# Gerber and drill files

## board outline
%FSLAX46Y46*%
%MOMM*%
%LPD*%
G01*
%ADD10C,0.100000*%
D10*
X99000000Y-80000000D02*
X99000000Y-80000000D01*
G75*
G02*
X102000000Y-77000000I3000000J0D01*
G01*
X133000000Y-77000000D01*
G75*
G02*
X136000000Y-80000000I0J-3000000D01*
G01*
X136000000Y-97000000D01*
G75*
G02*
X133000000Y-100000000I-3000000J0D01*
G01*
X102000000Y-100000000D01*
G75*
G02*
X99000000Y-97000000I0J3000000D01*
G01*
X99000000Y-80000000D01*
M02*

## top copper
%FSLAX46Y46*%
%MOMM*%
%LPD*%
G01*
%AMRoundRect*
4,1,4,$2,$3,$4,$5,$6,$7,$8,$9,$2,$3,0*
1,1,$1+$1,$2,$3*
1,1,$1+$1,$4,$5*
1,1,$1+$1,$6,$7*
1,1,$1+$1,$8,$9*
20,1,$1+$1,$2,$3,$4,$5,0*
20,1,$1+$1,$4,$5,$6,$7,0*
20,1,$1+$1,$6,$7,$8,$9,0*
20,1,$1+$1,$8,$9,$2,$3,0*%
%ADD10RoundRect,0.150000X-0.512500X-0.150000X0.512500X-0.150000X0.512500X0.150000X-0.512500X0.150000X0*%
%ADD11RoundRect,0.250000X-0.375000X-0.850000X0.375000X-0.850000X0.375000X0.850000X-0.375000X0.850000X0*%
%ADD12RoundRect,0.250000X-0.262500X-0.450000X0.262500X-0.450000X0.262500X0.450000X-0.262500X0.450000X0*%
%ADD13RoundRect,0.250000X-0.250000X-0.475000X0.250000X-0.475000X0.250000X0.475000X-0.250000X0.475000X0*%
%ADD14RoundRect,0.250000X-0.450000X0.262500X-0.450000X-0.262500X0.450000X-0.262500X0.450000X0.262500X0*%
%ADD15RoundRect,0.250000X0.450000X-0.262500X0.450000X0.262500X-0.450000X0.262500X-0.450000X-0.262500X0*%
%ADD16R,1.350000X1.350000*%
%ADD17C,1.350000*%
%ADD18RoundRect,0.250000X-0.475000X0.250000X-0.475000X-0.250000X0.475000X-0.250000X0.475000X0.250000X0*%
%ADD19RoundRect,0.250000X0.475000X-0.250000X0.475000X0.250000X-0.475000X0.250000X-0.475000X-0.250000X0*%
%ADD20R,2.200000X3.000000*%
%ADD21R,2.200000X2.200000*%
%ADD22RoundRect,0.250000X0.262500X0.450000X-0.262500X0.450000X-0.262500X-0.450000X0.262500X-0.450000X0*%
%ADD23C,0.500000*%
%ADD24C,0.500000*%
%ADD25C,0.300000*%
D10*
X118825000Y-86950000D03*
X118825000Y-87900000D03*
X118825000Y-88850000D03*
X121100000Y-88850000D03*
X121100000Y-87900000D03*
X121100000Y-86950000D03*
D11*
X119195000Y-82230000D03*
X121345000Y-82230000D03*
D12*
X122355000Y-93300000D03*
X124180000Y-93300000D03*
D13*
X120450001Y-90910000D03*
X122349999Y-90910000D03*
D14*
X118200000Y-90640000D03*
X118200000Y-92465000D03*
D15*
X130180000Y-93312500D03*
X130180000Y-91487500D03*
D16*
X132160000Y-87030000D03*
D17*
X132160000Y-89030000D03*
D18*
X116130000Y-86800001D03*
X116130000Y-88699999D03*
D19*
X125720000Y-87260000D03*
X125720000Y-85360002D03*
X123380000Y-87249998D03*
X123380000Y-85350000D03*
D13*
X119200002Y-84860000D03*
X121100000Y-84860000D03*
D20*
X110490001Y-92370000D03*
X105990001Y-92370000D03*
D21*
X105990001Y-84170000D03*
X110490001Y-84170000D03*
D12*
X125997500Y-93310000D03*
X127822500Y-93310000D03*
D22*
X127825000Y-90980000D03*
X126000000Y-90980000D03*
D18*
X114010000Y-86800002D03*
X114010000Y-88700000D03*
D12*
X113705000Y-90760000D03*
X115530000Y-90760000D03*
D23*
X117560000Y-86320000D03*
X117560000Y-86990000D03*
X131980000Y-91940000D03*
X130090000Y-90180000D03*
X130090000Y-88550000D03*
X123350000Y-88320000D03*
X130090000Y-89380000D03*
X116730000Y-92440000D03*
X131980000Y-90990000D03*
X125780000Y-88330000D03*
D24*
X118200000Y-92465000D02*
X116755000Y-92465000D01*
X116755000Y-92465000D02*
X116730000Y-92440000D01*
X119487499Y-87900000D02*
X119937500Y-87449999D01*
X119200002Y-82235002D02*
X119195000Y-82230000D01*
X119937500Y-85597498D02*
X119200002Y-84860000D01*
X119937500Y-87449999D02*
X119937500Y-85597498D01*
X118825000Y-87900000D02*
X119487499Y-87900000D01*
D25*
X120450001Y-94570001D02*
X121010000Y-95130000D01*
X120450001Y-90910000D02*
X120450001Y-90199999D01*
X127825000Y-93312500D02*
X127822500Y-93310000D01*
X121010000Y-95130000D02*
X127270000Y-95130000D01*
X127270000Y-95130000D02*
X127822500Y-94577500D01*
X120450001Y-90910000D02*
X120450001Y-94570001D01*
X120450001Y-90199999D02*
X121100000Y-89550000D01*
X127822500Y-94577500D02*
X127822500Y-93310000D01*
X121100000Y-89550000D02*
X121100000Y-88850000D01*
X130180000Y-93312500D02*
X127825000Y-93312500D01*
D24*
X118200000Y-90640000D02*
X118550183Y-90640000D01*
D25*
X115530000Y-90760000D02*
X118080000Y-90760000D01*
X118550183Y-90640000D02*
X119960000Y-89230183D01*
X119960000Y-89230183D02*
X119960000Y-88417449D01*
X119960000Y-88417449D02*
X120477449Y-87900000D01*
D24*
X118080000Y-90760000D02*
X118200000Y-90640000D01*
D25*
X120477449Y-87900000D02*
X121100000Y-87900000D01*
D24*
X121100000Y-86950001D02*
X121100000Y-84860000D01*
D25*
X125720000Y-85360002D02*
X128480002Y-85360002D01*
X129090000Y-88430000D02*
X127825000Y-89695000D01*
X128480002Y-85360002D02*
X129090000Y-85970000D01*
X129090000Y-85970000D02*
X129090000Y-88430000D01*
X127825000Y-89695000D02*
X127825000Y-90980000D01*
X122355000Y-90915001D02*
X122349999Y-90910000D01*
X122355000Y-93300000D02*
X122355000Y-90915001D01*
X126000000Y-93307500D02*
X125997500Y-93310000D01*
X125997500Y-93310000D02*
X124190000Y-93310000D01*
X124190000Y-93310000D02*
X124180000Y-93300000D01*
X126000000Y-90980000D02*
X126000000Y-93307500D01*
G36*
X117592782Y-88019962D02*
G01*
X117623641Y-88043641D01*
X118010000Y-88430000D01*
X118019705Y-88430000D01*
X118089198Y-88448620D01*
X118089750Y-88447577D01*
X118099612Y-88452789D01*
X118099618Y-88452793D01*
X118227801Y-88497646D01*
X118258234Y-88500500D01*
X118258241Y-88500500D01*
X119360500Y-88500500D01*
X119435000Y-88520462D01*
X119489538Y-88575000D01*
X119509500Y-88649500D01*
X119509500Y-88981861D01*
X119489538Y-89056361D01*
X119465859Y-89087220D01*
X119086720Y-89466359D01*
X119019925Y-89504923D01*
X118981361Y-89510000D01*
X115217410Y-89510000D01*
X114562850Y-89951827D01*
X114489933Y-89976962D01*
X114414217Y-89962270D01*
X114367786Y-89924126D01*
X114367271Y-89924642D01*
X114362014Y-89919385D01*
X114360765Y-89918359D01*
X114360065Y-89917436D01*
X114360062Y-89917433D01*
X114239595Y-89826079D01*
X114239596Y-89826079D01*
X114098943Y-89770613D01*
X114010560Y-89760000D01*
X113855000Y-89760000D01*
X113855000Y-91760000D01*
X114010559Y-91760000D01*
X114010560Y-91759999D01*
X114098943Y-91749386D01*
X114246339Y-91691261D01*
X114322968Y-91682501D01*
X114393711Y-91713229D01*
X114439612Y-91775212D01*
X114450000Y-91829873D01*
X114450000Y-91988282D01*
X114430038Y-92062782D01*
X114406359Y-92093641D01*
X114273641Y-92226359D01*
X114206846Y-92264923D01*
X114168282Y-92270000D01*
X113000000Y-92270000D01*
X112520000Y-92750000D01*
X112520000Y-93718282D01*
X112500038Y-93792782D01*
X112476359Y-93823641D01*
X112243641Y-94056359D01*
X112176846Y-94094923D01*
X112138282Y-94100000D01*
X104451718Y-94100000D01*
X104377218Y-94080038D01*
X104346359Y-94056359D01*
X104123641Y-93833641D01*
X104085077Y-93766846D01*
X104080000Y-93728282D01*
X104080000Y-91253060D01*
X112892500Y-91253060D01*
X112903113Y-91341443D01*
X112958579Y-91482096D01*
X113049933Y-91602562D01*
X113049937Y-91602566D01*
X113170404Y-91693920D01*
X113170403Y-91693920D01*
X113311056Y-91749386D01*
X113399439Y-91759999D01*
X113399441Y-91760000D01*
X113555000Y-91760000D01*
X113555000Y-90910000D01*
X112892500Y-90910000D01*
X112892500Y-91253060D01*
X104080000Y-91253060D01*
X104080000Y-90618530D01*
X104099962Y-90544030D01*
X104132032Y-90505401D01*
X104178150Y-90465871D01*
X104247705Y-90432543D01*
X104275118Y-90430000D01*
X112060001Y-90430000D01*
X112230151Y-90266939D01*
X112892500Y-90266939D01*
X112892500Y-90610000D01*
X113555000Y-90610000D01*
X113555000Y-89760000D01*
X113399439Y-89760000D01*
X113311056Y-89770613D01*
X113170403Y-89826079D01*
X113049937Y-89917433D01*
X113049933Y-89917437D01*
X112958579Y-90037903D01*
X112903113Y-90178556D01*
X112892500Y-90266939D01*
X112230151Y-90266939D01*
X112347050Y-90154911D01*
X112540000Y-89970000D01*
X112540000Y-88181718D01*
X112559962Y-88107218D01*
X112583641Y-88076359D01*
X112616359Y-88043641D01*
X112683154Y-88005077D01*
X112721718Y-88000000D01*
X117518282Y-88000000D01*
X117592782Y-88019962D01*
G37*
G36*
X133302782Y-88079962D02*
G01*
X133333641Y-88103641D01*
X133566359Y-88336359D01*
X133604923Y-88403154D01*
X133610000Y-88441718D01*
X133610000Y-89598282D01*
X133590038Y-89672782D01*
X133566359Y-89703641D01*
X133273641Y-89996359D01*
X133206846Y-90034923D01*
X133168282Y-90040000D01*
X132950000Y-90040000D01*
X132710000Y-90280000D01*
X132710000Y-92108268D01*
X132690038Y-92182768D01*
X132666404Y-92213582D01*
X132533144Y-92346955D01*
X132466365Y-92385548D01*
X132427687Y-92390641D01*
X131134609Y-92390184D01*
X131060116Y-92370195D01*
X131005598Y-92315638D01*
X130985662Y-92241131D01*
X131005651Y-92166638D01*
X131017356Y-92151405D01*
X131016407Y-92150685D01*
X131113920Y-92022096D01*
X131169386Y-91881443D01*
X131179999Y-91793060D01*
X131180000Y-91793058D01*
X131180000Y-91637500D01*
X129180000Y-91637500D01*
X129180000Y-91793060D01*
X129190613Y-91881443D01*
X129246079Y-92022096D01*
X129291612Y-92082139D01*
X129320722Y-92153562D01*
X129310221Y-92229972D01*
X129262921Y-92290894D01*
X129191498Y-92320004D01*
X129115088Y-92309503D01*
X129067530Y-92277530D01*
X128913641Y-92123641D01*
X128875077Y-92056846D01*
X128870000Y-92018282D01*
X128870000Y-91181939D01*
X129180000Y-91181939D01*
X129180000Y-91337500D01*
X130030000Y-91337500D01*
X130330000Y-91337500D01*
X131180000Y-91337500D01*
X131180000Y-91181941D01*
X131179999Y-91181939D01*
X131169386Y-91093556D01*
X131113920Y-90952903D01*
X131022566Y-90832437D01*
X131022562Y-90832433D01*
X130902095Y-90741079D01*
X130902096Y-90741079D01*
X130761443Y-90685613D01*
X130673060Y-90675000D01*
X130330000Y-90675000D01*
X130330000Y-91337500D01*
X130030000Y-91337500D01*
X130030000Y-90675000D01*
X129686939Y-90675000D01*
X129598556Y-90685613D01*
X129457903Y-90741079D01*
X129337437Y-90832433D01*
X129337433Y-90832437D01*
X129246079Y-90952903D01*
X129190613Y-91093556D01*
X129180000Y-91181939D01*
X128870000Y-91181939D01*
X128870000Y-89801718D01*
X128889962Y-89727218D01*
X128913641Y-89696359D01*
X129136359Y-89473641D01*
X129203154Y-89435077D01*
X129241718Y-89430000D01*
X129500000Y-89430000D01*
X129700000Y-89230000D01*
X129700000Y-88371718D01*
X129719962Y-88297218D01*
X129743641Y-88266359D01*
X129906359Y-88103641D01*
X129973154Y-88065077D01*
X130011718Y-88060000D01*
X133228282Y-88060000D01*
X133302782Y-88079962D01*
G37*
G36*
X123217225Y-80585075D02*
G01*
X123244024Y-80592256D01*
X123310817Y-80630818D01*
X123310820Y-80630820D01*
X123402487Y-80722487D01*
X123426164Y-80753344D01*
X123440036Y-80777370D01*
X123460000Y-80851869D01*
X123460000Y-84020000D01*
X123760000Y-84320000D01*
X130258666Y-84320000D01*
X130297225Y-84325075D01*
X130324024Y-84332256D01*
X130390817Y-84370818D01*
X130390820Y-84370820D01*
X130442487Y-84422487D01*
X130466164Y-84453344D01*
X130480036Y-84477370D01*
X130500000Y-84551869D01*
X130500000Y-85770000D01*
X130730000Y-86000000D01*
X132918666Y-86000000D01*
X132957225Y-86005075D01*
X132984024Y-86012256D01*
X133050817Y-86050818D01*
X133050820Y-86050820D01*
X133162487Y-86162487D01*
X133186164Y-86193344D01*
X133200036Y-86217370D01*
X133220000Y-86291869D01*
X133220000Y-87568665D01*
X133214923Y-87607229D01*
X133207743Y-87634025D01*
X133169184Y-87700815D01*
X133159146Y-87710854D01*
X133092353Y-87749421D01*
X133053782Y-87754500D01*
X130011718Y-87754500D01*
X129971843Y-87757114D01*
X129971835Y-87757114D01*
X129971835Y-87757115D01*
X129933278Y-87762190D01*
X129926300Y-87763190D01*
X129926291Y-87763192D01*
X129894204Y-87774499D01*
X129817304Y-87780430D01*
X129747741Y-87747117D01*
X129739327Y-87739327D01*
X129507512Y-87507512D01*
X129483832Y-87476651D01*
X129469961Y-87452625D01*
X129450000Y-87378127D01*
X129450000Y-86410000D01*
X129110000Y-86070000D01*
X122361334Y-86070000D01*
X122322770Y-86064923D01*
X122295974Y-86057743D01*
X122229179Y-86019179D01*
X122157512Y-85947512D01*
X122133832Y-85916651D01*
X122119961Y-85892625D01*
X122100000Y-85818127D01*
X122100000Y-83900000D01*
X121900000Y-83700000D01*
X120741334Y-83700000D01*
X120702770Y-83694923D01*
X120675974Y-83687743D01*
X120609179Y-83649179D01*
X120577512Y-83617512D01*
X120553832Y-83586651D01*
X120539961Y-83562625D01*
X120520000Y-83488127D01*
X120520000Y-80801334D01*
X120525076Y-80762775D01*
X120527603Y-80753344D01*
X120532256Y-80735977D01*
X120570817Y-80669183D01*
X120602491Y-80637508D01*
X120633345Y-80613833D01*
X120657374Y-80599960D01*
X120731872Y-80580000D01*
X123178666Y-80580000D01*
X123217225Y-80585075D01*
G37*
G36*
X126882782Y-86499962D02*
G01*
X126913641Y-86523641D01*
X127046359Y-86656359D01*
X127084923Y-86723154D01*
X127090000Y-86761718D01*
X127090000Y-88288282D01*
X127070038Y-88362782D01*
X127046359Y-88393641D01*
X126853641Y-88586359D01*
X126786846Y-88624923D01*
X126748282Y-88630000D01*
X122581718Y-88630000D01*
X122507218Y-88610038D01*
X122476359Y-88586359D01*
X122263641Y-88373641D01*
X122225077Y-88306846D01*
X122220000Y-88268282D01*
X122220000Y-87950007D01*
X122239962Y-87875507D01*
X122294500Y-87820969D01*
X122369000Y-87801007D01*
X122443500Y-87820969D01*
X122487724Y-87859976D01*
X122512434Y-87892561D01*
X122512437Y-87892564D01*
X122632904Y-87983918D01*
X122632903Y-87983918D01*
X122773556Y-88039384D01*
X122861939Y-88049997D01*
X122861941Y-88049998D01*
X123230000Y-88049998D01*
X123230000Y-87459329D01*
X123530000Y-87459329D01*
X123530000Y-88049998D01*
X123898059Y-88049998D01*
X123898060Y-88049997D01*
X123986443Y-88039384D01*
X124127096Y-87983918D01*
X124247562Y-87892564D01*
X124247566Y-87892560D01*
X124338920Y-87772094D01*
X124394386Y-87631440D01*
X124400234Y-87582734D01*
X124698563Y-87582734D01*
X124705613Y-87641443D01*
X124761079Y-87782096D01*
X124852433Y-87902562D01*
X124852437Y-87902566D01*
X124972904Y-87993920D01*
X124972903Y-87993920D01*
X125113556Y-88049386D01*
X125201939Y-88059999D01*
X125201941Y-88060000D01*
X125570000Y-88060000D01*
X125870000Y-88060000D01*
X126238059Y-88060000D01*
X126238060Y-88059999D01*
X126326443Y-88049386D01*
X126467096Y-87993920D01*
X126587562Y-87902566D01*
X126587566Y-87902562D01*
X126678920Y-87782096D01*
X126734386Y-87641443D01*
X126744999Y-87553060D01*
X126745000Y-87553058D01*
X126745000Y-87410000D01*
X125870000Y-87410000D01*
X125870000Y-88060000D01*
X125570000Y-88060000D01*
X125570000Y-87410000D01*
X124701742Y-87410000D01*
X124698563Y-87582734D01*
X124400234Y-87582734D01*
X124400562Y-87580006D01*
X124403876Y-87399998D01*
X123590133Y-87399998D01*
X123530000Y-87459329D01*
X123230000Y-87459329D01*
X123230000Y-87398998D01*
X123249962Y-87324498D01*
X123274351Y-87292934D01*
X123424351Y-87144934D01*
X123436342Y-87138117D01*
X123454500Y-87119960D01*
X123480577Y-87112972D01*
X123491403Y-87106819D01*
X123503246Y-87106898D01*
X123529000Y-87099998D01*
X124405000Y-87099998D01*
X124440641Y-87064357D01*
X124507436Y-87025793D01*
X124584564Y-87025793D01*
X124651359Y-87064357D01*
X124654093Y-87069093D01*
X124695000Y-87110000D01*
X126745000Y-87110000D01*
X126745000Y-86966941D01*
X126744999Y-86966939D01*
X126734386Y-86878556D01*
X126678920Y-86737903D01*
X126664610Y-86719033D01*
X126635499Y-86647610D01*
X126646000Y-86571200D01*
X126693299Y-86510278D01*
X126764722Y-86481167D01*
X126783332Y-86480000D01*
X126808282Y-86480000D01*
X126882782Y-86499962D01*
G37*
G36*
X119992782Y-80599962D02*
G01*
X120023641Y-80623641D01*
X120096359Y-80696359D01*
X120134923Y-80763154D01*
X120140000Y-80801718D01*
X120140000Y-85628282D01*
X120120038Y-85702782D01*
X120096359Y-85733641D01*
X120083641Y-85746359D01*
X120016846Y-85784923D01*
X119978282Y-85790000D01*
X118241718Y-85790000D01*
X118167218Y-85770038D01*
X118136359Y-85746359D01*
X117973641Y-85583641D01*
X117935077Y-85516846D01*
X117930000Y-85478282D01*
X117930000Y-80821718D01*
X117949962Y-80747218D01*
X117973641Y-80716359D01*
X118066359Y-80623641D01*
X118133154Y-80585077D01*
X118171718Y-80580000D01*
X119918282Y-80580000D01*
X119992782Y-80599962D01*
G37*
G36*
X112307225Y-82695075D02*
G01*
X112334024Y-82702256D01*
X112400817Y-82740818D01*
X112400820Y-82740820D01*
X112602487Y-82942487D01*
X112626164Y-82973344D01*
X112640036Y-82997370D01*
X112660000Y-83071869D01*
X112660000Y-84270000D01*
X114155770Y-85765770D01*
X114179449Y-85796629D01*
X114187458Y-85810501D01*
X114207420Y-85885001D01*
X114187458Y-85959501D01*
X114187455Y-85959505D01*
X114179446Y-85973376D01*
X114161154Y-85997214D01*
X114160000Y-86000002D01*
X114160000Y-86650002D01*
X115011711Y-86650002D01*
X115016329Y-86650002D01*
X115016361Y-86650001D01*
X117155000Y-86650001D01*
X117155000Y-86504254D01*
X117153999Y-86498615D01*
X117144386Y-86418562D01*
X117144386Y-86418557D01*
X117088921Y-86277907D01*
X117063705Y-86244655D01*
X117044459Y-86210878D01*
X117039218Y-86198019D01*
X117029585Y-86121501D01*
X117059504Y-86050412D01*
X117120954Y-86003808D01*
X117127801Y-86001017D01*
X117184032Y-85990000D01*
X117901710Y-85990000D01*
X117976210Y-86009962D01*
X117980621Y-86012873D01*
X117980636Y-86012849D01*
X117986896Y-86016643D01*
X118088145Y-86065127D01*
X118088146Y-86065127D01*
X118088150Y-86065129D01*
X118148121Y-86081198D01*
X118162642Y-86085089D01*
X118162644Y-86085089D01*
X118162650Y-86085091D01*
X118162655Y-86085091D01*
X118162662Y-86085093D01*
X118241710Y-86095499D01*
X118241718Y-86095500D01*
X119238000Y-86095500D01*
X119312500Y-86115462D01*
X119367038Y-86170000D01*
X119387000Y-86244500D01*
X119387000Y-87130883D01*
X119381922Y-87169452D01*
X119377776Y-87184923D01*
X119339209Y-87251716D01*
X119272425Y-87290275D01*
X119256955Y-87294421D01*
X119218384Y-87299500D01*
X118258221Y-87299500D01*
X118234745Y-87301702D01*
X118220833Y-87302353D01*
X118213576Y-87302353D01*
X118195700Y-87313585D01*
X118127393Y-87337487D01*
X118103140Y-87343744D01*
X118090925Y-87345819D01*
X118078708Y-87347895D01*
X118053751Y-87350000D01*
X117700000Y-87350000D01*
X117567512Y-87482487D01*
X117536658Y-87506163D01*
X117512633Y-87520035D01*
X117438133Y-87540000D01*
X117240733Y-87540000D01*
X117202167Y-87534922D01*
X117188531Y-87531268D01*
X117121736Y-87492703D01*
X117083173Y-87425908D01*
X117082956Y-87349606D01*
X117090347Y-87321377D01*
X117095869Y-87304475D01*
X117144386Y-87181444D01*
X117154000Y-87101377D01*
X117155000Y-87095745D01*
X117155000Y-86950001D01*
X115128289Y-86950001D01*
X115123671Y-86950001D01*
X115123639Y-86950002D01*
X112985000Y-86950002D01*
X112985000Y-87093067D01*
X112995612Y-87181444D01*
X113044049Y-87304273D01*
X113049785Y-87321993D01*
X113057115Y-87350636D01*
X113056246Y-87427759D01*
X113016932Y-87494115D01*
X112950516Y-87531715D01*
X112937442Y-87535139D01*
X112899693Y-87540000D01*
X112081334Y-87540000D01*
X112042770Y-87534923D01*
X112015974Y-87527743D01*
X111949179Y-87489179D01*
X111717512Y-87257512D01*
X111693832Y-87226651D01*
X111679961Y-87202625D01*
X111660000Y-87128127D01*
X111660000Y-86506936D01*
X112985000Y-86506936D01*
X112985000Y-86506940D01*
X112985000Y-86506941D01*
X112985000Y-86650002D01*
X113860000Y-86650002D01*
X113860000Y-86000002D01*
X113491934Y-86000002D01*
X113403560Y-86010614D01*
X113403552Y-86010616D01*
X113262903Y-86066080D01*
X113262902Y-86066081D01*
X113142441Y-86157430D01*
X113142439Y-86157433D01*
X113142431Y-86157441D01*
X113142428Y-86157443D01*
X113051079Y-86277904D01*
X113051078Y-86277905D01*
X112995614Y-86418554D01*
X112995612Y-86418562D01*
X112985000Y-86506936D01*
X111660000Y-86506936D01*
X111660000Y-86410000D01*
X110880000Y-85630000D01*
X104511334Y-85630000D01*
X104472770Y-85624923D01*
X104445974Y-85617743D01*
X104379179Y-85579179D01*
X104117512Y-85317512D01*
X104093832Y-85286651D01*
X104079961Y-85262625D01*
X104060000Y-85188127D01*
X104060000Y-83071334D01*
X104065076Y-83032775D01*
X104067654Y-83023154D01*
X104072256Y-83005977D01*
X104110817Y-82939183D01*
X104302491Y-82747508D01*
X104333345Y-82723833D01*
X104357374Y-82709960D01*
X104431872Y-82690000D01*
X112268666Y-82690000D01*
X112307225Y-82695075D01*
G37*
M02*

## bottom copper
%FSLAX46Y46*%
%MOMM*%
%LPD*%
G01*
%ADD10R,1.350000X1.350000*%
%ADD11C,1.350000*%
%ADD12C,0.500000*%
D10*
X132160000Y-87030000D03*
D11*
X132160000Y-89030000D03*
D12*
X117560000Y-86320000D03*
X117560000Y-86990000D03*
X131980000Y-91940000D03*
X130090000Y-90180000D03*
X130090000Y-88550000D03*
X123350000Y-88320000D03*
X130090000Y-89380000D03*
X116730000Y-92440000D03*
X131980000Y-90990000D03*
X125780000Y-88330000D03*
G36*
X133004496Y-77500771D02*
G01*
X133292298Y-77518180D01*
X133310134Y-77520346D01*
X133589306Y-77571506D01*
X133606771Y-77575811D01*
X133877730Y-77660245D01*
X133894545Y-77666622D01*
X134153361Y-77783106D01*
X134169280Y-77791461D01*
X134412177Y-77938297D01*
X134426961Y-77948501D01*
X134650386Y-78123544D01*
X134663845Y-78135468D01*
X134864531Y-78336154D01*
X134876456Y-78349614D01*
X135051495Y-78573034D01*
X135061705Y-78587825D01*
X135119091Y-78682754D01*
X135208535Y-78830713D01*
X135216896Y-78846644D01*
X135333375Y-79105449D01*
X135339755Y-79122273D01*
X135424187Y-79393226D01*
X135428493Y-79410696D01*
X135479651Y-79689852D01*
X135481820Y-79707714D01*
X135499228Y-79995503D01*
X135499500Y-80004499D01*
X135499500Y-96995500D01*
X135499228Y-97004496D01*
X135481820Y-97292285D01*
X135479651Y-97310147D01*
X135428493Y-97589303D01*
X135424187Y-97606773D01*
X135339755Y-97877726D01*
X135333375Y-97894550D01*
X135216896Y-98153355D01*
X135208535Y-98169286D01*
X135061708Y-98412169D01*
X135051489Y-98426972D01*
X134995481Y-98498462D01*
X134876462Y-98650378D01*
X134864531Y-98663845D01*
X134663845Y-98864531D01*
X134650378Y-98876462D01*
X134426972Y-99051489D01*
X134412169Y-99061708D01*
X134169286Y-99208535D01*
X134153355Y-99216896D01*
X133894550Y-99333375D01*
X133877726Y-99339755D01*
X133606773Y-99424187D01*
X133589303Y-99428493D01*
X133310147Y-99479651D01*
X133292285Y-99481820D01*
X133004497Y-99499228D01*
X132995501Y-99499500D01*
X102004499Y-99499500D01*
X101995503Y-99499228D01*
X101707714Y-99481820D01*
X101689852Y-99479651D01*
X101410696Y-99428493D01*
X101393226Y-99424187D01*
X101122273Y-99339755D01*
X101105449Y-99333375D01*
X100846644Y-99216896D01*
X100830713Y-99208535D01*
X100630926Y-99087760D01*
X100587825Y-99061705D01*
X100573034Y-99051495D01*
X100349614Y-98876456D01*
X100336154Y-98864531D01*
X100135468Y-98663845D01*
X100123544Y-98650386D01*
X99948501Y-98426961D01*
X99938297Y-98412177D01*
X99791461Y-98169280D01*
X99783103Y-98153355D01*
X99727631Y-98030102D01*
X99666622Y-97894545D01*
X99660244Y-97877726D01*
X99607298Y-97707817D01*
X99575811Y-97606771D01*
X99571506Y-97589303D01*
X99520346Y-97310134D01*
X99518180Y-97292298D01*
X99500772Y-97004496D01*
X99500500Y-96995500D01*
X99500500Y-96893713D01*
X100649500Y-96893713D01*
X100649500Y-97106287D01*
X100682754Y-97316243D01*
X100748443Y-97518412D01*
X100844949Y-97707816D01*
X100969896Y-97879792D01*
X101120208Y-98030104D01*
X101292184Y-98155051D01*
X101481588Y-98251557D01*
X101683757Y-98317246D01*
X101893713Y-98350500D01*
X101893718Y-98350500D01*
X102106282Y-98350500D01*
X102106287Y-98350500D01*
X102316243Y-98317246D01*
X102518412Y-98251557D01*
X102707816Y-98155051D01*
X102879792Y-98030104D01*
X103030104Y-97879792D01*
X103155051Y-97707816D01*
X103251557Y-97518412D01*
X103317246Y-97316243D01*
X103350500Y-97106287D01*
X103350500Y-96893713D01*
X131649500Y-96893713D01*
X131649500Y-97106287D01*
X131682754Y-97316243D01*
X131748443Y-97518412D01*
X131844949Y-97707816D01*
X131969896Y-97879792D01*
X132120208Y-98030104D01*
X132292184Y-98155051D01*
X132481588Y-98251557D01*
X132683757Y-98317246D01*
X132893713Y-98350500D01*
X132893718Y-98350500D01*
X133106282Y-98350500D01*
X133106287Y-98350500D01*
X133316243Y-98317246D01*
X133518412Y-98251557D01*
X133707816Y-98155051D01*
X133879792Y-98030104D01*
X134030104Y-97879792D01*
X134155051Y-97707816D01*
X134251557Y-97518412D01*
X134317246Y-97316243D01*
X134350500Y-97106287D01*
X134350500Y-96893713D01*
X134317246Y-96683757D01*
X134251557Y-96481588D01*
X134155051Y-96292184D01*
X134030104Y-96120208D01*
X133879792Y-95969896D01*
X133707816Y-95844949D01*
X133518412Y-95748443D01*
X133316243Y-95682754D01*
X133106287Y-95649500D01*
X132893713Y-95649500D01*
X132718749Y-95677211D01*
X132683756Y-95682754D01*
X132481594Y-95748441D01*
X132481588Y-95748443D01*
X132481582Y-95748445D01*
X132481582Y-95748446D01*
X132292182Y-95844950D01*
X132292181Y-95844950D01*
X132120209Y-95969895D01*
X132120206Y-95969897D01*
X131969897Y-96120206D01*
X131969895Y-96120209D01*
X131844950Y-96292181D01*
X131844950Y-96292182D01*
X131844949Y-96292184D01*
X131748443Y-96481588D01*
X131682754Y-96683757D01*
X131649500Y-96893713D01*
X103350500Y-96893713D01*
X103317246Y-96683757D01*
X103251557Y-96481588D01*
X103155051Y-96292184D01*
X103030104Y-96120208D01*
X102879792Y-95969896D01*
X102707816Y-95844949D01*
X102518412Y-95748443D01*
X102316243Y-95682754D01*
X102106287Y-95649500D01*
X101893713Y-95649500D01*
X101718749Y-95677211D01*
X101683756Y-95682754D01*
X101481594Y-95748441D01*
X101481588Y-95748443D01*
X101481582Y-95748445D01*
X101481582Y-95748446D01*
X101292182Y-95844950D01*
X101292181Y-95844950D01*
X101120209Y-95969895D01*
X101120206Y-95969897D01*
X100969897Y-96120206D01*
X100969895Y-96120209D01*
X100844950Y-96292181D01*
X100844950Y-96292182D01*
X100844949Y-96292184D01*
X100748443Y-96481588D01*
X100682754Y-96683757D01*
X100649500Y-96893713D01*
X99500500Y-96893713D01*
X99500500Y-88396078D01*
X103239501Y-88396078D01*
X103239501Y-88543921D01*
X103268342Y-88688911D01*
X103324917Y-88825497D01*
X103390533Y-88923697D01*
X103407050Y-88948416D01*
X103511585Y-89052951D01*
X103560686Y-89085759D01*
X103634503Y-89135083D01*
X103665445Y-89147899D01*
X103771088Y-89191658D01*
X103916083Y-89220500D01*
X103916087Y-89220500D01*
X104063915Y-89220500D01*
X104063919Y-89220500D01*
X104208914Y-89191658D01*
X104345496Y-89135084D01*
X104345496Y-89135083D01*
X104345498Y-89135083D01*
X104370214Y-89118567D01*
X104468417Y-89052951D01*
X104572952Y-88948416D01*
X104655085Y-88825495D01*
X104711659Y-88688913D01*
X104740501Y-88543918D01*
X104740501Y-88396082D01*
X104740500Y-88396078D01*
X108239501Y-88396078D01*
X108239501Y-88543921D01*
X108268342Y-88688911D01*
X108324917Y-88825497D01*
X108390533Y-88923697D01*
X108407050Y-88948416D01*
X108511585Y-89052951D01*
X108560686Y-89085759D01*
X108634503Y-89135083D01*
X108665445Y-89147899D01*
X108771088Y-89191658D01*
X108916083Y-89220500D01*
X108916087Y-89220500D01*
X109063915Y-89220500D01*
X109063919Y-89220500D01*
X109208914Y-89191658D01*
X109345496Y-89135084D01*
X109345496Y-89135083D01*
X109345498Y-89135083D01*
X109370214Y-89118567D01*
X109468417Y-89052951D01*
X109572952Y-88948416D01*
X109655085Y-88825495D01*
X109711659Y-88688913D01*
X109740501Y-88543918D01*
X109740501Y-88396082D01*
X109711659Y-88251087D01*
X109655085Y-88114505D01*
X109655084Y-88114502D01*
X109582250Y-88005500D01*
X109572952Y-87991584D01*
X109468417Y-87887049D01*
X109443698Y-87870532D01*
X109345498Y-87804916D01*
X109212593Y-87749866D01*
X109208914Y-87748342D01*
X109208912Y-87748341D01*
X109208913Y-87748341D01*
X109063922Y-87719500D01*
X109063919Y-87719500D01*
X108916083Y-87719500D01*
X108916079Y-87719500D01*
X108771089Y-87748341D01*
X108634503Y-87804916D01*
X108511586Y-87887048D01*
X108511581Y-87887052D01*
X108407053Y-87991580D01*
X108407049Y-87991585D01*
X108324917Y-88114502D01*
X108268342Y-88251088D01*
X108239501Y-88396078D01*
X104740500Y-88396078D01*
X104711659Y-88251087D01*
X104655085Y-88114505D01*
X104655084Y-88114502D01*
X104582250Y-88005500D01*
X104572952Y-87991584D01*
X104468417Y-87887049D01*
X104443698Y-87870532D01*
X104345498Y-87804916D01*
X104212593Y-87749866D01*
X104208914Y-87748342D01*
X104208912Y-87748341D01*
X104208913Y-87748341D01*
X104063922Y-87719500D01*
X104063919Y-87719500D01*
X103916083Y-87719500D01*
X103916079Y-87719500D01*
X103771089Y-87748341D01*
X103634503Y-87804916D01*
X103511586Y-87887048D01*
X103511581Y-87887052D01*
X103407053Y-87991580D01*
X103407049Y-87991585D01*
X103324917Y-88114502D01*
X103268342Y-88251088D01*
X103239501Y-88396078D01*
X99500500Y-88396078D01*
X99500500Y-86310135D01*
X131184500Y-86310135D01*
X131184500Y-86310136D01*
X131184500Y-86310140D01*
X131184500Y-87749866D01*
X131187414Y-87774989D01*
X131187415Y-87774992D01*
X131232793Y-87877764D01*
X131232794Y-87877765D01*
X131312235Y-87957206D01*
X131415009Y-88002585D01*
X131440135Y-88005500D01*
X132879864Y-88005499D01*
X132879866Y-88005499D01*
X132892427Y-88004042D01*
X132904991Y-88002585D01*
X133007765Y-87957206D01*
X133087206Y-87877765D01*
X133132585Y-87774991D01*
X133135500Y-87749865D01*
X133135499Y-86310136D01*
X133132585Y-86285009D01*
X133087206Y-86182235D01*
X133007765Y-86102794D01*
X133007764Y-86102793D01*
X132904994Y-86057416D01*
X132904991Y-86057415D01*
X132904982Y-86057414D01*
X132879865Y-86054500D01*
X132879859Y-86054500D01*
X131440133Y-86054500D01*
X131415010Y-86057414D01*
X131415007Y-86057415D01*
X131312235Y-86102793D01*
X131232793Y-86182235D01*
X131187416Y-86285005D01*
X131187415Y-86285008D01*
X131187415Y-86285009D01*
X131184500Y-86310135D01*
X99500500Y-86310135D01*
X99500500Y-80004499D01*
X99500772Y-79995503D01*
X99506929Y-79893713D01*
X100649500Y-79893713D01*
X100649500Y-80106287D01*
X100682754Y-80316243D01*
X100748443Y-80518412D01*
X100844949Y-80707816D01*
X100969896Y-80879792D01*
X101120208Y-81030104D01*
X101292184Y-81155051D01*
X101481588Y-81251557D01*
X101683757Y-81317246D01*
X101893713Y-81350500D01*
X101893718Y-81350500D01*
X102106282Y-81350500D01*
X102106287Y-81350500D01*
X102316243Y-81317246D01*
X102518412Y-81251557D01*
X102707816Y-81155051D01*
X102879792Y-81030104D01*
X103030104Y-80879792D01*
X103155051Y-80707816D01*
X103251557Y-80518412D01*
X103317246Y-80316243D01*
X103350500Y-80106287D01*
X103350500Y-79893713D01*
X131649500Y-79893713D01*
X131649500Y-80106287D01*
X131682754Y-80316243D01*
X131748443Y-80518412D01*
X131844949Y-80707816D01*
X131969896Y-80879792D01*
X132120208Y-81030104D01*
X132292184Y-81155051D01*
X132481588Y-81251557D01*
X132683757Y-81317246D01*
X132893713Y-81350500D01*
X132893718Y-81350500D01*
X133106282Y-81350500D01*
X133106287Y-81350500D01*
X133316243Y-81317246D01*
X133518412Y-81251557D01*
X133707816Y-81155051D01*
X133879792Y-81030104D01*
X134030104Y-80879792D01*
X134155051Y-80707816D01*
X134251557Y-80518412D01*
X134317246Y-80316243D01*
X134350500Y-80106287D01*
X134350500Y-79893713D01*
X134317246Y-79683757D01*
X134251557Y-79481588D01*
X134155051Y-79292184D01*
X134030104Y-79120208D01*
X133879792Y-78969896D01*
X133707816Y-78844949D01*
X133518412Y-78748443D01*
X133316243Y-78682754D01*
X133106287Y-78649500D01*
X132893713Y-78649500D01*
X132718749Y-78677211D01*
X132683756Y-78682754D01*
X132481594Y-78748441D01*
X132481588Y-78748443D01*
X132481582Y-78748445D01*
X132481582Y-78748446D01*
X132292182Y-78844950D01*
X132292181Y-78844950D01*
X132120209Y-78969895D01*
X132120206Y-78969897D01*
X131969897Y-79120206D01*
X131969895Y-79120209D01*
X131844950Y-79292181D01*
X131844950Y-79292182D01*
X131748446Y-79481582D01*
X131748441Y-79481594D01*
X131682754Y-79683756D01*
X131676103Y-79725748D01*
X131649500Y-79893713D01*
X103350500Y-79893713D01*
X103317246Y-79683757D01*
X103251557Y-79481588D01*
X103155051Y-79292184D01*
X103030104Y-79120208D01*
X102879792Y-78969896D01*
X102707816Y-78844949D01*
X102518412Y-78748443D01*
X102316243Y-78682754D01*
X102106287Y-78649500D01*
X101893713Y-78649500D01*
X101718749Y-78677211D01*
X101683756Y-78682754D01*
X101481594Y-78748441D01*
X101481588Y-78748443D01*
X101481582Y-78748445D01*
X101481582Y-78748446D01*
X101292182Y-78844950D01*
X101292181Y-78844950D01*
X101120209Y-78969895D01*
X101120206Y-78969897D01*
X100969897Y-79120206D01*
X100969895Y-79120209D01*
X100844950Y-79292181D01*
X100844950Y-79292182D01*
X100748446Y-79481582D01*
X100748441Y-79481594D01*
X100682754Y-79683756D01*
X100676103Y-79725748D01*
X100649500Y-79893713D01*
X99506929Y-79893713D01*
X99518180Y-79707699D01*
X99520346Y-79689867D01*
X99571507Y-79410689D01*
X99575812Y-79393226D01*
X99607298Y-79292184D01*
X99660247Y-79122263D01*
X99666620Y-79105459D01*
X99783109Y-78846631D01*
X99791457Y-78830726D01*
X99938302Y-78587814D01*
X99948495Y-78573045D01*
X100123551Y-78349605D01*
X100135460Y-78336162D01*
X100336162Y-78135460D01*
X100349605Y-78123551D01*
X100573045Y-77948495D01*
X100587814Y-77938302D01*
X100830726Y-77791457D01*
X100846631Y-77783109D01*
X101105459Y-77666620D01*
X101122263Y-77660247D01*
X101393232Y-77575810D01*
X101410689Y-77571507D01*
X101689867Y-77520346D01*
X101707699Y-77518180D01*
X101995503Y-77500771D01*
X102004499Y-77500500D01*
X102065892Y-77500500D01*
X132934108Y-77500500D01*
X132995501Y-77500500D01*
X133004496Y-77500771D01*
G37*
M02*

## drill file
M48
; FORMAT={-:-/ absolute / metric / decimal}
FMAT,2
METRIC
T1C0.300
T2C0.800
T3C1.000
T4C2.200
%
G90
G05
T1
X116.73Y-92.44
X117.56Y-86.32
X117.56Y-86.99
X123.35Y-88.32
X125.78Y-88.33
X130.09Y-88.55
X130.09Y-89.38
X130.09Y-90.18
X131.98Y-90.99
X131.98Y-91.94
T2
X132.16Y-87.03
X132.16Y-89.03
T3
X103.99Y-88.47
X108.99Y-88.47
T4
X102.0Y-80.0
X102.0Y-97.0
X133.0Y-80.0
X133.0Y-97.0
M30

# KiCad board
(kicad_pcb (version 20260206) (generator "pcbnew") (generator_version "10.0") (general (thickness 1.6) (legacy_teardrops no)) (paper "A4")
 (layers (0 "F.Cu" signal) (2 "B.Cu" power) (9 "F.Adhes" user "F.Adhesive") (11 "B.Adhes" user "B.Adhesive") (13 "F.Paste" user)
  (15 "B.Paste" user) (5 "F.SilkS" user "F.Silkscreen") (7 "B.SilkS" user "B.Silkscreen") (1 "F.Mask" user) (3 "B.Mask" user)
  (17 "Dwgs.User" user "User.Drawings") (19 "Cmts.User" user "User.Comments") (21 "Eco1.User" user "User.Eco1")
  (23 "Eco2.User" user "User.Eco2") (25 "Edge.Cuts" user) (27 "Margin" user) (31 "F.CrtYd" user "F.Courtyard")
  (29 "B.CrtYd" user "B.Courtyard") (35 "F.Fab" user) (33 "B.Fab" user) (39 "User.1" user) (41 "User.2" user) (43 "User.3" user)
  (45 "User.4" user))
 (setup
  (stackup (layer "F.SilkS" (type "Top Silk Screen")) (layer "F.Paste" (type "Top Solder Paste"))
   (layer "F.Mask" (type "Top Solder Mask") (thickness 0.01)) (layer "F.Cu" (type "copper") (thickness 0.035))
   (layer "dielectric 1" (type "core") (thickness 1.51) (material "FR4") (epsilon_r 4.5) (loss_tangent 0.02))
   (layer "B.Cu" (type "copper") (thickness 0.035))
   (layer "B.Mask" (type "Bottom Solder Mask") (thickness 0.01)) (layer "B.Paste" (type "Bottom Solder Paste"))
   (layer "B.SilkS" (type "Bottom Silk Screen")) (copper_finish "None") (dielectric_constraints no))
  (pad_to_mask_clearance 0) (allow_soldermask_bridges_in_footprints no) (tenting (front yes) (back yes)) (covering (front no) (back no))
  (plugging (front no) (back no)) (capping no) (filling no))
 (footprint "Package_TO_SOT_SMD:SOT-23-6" (layer "F.Cu") (at 119.9625 87.9)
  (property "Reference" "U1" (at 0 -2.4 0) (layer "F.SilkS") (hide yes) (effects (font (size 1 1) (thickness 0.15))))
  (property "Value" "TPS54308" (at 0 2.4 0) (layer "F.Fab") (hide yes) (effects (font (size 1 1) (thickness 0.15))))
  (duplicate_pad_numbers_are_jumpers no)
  (pad "1" smd roundrect (at -1.1375 -0.95) (size 1.325 0.6) (layers "F.Cu" "F.Mask" "F.Paste") (roundrect_rratio 0.25) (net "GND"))
  (pad "2" smd roundrect (at -1.1375 0) (size 1.325 0.6) (layers "F.Cu" "F.Mask" "F.Paste") (roundrect_rratio 0.25) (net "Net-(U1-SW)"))
  (pad "3" smd roundrect (at -1.1375 0.95) (size 1.325 0.6) (layers "F.Cu" "F.Mask" "F.Paste") (roundrect_rratio 0.25) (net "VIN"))
  (pad "4" smd roundrect (at 1.1375 0.95) (size 1.325 0.6) (layers "F.Cu" "F.Mask" "F.Paste") (roundrect_rratio 0.25) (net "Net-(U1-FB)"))
  (pad "5" smd roundrect (at 1.1375 0) (size 1.325 0.6) (layers "F.Cu" "F.Mask" "F.Paste") (roundrect_rratio 0.25) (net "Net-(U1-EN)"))
  (pad "6" smd roundrect (at 1.1375 -0.95) (size 1.325 0.6) (layers "F.Cu" "F.Mask" "F.Paste") (roundrect_rratio 0.25) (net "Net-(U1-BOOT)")))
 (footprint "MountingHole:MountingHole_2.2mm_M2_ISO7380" (layer "F.Cu") (at 133 80)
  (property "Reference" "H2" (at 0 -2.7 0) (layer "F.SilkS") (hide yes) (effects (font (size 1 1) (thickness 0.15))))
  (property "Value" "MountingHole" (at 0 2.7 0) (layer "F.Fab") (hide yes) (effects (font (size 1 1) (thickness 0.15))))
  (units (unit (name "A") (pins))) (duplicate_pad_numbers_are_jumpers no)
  (pad "" np_thru_hole circle (at 0 0) (size 2.2 2.2) (drill 2.2) (layers "*.Cu" "*.Mask")))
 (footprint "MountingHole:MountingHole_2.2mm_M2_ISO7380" (layer "F.Cu") (at 102 80)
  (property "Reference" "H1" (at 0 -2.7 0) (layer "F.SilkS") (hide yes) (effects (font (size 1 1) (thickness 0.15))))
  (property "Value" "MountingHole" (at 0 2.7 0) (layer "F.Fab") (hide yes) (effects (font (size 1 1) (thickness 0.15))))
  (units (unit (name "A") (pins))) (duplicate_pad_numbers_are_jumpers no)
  (pad "" np_thru_hole circle (at 0 0) (size 2.2 2.2) (drill 2.2) (layers "*.Cu" "*.Mask")))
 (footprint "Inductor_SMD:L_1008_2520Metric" (layer "F.Cu") (at 120.27 82.23)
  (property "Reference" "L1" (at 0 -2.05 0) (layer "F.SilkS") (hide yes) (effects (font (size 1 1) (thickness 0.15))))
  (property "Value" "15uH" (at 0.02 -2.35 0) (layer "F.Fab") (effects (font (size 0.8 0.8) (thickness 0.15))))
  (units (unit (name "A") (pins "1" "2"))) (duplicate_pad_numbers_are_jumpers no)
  (pad "1" smd roundrect (at -1.075 0) (size 1.25 2.2) (layers "F.Cu" "F.Mask" "F.Paste") (roundrect_rratio 0.2) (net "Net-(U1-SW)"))
  (pad "2" smd roundrect (at 1.075 0) (size 1.25 2.2) (layers "F.Cu" "F.Mask" "F.Paste") (roundrect_rratio 0.2) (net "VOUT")))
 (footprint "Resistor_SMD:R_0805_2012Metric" (layer "F.Cu") (at 123.2675 93.3)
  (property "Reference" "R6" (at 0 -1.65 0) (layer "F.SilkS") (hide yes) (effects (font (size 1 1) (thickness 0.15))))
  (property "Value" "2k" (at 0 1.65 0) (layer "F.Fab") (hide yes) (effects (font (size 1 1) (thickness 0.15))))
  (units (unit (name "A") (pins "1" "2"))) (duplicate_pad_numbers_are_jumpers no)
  (pad "1" smd roundrect (at -0.9125 0) (size 1.025 1.4) (layers "F.Cu" "F.Mask" "F.Paste") (roundrect_rratio 0.243902)
   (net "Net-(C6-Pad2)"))
  (pad "2" smd roundrect (at 0.9125 0) (size 1.025 1.4) (layers "F.Cu" "F.Mask" "F.Paste") (roundrect_rratio 0.243902) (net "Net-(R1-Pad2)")))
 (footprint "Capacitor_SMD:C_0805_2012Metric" (layer "F.Cu") (at 121.4 90.91)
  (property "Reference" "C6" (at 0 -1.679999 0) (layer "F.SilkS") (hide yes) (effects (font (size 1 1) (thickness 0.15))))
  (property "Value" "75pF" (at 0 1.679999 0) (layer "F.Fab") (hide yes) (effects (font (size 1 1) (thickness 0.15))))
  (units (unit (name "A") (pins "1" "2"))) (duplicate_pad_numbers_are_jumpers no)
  (pad "1" smd roundrect (at -0.949999 0) (size 1 1.45) (layers "F.Cu" "F.Mask" "F.Paste") (roundrect_rratio 0.25) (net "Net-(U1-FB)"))
  (pad "2" smd roundrect (at 0.949999 0) (size 1 1.45) (layers "F.Cu" "F.Mask" "F.Paste") (roundrect_rratio 0.25) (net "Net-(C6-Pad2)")))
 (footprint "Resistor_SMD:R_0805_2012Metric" (layer "F.Cu") (at 118.2 91.5525 -90)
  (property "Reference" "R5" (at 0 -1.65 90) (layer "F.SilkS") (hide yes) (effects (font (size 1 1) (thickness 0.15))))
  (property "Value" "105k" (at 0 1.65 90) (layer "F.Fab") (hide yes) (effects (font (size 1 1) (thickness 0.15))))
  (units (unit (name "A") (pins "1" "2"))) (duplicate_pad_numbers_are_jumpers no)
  (pad "1" smd roundrect (at -0.9125 0 270) (size 1.025 1.4) (layers "F.Cu" "F.Mask" "F.Paste") (roundrect_rratio 0.243902)
   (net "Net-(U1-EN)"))
  (pad "2" smd roundrect (at 0.9125 0 270) (size 1.025 1.4) (layers "F.Cu" "F.Mask" "F.Paste") (roundrect_rratio 0.243902) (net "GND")))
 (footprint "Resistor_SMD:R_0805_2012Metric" (layer "F.Cu") (at 130.18 92.4 90)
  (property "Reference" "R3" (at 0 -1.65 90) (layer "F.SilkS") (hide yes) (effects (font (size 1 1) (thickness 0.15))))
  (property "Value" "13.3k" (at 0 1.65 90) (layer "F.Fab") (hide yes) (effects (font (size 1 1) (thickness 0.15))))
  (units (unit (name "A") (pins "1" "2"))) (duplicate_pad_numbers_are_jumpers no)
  (pad "1" smd roundrect (at -0.9125 0 90) (size 1.025 1.4) (layers "F.Cu" "F.Mask" "F.Paste") (roundrect_rratio 0.243902)
   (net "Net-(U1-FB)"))
  (pad "2" smd roundrect (at 0.9125 0 90) (size 1.025 1.4) (layers "F.Cu" "F.Mask" "F.Paste") (roundrect_rratio 0.243902) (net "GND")
   (zone_connect 1)))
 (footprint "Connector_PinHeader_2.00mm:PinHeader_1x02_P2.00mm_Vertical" (layer "F.Cu") (at 132.16 87.03)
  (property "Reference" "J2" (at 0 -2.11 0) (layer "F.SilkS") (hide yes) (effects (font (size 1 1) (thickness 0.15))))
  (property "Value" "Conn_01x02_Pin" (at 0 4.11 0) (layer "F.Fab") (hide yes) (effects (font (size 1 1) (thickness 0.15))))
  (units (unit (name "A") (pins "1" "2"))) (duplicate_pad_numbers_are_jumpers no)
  (pad "1" thru_hole rect (at 0 0) (size 1.35 1.35) (drill 0.8) (layers "*.Cu" "*.Mask") (remove_unused_layers no) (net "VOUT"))
  (pad "2" thru_hole circle (at 0 2) (size 1.35 1.35) (drill 0.8) (layers "*.Cu" "*.Mask") (remove_unused_layers no) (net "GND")))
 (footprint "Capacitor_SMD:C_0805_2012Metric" (layer "F.Cu") (at 116.13 87.75 -90)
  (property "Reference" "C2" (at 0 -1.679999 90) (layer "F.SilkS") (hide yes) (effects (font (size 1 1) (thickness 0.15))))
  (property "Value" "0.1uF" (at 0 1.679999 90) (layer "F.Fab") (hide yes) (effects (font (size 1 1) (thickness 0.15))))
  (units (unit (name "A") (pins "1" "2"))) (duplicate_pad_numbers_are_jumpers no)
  (pad "1" smd roundrect (at -0.949999 0 270) (size 1 1.45) (layers "F.Cu" "F.Mask" "F.Paste") (roundrect_rratio 0.25) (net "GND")
   (zone_connect 1))
  (pad "2" smd roundrect (at 0.949999 0 270) (size 1 1.45) (layers "F.Cu" "F.Mask" "F.Paste") (roundrect_rratio 0.25) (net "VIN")))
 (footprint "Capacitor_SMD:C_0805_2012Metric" (layer "F.Cu") (at 125.72 86.310001 90)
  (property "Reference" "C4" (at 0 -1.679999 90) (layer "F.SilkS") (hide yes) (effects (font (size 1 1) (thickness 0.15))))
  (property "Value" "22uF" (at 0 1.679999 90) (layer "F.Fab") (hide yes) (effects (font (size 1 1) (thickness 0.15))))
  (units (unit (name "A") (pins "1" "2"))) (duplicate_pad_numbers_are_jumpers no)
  (pad "1" smd roundrect (at -0.949999 0 90) (size 1 1.45) (layers "F.Cu" "F.Mask" "F.Paste") (roundrect_rratio 0.25) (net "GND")
   (zone_connect 1))
  (pad "2" smd roundrect (at 0.949999 0 90) (size 1 1.45) (layers "F.Cu" "F.Mask" "F.Paste") (roundrect_rratio 0.25) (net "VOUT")))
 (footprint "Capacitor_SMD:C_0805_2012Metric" (layer "F.Cu") (at 123.38 86.299999 90)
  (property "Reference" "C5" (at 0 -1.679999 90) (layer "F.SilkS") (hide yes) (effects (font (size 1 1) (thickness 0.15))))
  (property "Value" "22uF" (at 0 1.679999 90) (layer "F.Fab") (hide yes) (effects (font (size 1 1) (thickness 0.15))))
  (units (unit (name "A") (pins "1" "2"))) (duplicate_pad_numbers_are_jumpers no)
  (pad "1" smd roundrect (at -0.949999 0 90) (size 1 1.45) (layers "F.Cu" "F.Mask" "F.Paste") (roundrect_rratio 0.25) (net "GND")
   (zone_connect 1))
  (pad "2" smd roundrect (at 0.949999 0 90) (size 1 1.45) (layers "F.Cu" "F.Mask" "F.Paste") (roundrect_rratio 0.25) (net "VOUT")))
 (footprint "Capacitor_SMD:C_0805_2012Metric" (layer "F.Cu") (at 120.150001 84.86)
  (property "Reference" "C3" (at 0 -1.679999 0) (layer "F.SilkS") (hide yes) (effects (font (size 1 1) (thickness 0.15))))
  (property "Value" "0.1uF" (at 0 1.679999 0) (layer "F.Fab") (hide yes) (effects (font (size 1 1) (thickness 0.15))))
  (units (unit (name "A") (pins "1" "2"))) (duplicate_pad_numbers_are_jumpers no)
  (pad "1" smd roundrect (at -0.949999 0) (size 1 1.45) (layers "F.Cu" "F.Mask" "F.Paste") (roundrect_rratio 0.25) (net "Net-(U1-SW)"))
  (pad "2" smd roundrect (at 0.949999 0) (size 1 1.45) (layers "F.Cu" "F.Mask" "F.Paste") (roundrect_rratio 0.25) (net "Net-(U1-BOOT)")))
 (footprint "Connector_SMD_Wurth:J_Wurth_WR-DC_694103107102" (layer "F.Cu") (at 106.490001 88.47 180)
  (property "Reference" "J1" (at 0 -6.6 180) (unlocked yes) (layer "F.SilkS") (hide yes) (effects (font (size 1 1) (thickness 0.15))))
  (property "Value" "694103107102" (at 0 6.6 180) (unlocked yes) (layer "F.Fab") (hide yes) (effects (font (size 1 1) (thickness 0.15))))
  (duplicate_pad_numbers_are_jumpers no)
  (pad "" np_thru_hole circle (at -2.5 0 270) (size 1 1) (drill 1) (layers "*.Cu" "*.Mask"))
  (pad "" np_thru_hole circle (at 2.5 0 270) (size 1 1) (drill 1) (layers "*.Cu" "*.Mask"))
  (pad "1" smd rect (at -4 -3.9 180) (size 2.2 3) (layers "F.Cu" "F.Mask" "F.Paste") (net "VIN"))
  (pad "1" smd rect (at 0.5 -3.9 180) (size 2.2 3) (layers "F.Cu" "F.Mask" "F.Paste") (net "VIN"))
  (pad "2" smd rect (at 0.5 4.3 270) (size 2.2 2.2) (layers "F.Cu" "F.Mask" "F.Paste") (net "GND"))
  (pad "3" smd rect (at -4 4.3 270) (size 2.2 2.2) (layers "F.Cu" "F.Mask" "F.Paste") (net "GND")))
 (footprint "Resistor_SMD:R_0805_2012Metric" (layer "F.Cu") (at 126.91 93.31)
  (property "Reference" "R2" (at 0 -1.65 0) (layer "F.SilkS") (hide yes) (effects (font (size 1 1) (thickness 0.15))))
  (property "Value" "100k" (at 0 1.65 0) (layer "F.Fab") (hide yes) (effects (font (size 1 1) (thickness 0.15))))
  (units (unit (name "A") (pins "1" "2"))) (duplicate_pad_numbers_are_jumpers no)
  (pad "1" smd roundrect (at -0.9125 0) (size 1.025 1.4) (layers "F.Cu" "F.Mask" "F.Paste") (roundrect_rratio 0.243902)
   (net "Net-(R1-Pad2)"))
  (pad "2" smd roundrect (at 0.9125 0) (size 1.025 1.4) (layers "F.Cu" "F.Mask" "F.Paste") (roundrect_rratio 0.243902) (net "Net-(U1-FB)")))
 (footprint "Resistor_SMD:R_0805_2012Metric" (layer "F.Cu") (at 126.9125 90.98 180)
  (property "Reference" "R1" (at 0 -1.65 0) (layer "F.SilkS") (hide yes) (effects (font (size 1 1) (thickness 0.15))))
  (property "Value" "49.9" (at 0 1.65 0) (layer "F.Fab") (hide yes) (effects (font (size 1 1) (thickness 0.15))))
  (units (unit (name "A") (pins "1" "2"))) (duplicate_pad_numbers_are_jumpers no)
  (pad "1" smd roundrect (at -0.9125 0 180) (size 1.025 1.4) (layers "F.Cu" "F.Mask" "F.Paste") (roundrect_rratio 0.243902) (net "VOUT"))
  (pad "2" smd roundrect (at 0.9125 0 180) (size 1.025 1.4) (layers "F.Cu" "F.Mask" "F.Paste") (roundrect_rratio 0.243902)
   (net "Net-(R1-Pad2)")))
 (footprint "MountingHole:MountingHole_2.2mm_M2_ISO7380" (layer "F.Cu") (at 133 97)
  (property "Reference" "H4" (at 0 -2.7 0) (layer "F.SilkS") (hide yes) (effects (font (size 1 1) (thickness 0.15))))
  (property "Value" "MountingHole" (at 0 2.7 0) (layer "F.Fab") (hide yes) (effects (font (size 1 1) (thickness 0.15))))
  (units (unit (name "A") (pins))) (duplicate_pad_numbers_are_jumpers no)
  (pad "" np_thru_hole circle (at 0 0) (size 2.2 2.2) (drill 2.2) (layers "*.Cu" "*.Mask")))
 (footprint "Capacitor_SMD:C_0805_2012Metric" (layer "F.Cu") (at 114.01 87.750001 -90)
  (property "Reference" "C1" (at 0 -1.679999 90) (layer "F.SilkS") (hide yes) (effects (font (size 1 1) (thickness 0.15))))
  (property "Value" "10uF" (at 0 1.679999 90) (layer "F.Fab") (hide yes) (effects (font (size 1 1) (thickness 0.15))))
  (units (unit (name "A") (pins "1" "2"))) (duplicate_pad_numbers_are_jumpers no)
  (pad "1" smd roundrect (at -0.949999 0 270) (size 1 1.45) (layers "F.Cu" "F.Mask" "F.Paste") (roundrect_rratio 0.25) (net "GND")
   (zone_connect 1))
  (pad "2" smd roundrect (at 0.949999 0 270) (size 1 1.45) (layers "F.Cu" "F.Mask" "F.Paste") (roundrect_rratio 0.25) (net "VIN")))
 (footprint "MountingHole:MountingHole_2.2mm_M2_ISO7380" (layer "F.Cu") (at 102 97)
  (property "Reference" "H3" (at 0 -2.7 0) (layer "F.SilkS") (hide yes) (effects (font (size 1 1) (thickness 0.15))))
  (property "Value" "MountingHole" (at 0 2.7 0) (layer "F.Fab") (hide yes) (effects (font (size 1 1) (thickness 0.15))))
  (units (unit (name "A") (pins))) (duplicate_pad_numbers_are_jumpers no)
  (pad "" np_thru_hole circle (at 0 0) (size 2.2 2.2) (drill 2.2) (layers "*.Cu" "*.Mask")))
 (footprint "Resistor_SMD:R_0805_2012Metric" (layer "F.Cu") (at 114.6175 90.76)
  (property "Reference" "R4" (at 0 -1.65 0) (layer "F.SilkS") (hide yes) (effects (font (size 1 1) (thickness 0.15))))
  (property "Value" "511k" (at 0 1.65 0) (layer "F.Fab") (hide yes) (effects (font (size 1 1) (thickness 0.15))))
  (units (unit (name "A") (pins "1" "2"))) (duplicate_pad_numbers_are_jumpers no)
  (pad "1" smd roundrect (at -0.9125 0) (size 1.025 1.4) (layers "F.Cu" "F.Mask" "F.Paste") (roundrect_rratio 0.243902) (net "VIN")
   (zone_connect 1))
  (pad "2" smd roundrect (at 0.9125 0) (size 1.025 1.4) (layers "F.Cu" "F.Mask" "F.Paste") (roundrect_rratio 0.243902) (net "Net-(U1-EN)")))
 (gr_rect (start 99 77) (end 136 100) (radius 3) (stroke (width 0.1) (type solid)) (fill no) (layer "Edge.Cuts"))
 (segment (start 118.2 92.465) (end 116.755 92.465) (width 0.5) (layer "F.Cu") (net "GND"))
 (segment (start 116.755 92.465) (end 116.73 92.44) (width 0.5) (layer "F.Cu") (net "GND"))
 (via (at 117.56 86.32) (size 0.5) (drill 0.3) (layers "F.Cu" "B.Cu") (free yes) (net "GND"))
 (via (at 117.56 86.99) (size 0.5) (drill 0.3) (layers "F.Cu" "B.Cu") (free yes) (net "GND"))
 (via (at 131.98 91.94) (size 0.5) (drill 0.3) (layers "F.Cu" "B.Cu") (free yes) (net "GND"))
 (via (at 130.09 90.18) (size 0.5) (drill 0.3) (layers "F.Cu" "B.Cu") (free yes) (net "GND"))
 (via (at 130.09 88.55) (size 0.5) (drill 0.3) (layers "F.Cu" "B.Cu") (free yes) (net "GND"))
 (via (at 123.35 88.32) (size 0.5) (drill 0.3) (layers "F.Cu" "B.Cu") (free yes) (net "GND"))
 (via (at 130.09 89.38) (size 0.5) (drill 0.3) (layers "F.Cu" "B.Cu") (free yes) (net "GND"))
 (via (at 116.73 92.44) (size 0.5) (drill 0.3) (layers "F.Cu" "B.Cu") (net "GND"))
 (via (at 131.98 90.99) (size 0.5) (drill 0.3) (layers "F.Cu" "B.Cu") (free yes) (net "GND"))
 (via (at 125.78 88.33) (size 0.5) (drill 0.3) (layers "F.Cu" "B.Cu") (free yes) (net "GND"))
 (segment (start 119.487499 87.9) (end 119.9375 87.449999) (width 0.5) (layer "F.Cu") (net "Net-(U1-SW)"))
 (segment (start 119.200002 82.235002) (end 119.195 82.23) (width 0.5) (layer "F.Cu") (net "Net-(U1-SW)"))
 (segment (start 119.9375 85.597498) (end 119.200002 84.86) (width 0.5) (layer "F.Cu") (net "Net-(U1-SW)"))
 (segment (start 119.9375 87.449999) (end 119.9375 85.597498) (width 0.5) (layer "F.Cu") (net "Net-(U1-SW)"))
 (segment (start 118.825 87.9) (end 119.487499 87.9) (width 0.5) (layer "F.Cu") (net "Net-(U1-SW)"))
 (segment (start 120.450001 94.570001) (end 121.01 95.13) (width 0.3) (layer "F.Cu") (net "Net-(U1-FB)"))
 (segment (start 120.450001 90.91) (end 120.450001 90.199999) (width 0.3) (layer "F.Cu") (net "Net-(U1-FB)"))
 (segment (start 127.825 93.3125) (end 127.8225 93.31) (width 0.3) (layer "F.Cu") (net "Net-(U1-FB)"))
 (segment (start 121.01 95.13) (end 127.27 95.13) (width 0.3) (layer "F.Cu") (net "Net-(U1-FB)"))
 (segment (start 127.27 95.13) (end 127.8225 94.5775) (width 0.3) (layer "F.Cu") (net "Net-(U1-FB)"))
 (segment (start 120.450001 90.91) (end 120.450001 94.570001) (width 0.3) (layer "F.Cu") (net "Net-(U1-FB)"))
 (segment (start 120.450001 90.199999) (end 121.1 89.55) (width 0.3) (layer "F.Cu") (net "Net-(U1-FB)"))
 (segment (start 127.8225 94.5775) (end 127.8225 93.31) (width 0.3) (layer "F.Cu") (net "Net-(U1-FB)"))
 (segment (start 121.1 89.55) (end 121.1 88.85) (width 0.3) (layer "F.Cu") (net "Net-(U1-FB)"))
 (segment (start 130.18 93.3125) (end 127.825 93.3125) (width 0.3) (layer "F.Cu") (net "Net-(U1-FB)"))
 (segment (start 118.2 90.64) (end 118.550183 90.64) (width 0.5) (layer "F.Cu") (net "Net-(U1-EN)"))
 (segment (start 115.53 90.76) (end 118.08 90.76) (width 0.3) (layer "F.Cu") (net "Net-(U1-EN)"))
 (segment (start 118.550183 90.64) (end 119.96 89.230183) (width 0.3) (layer "F.Cu") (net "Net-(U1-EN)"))
 (segment (start 119.96 89.230183) (end 119.96 88.417449) (width 0.3) (layer "F.Cu") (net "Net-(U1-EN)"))
 (segment (start 119.96 88.417449) (end 120.477449 87.9) (width 0.3) (layer "F.Cu") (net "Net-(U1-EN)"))
 (segment (start 118.08 90.76) (end 118.2 90.64) (width 0.5) (layer "F.Cu") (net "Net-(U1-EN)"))
 (segment (start 120.477449 87.9) (end 121.1 87.9) (width 0.3) (layer "F.Cu") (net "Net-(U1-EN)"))
 (segment (start 121.1 86.950001) (end 121.1 84.86) (width 0.5) (layer "F.Cu") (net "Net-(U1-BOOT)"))
 (segment (start 125.72 85.360002) (end 128.480002 85.360002) (width 0.3) (layer "F.Cu") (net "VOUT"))
 (segment (start 129.09 88.43) (end 127.825 89.695) (width 0.3) (layer "F.Cu") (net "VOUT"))
 (segment (start 128.480002 85.360002) (end 129.09 85.97) (width 0.3) (layer "F.Cu") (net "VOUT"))
 (segment (start 129.09 85.97) (end 129.09 88.43) (width 0.3) (layer "F.Cu") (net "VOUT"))
 (segment (start 127.825 89.695) (end 127.825 90.98) (width 0.3) (layer "F.Cu") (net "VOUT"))
 (segment (start 122.355 90.915001) (end 122.349999 90.91) (width 0.3) (layer "F.Cu") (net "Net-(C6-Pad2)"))
 (segment (start 122.355 93.3) (end 122.355 90.915001) (width 0.3) (layer "F.Cu") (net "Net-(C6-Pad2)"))
 (segment (start 126 93.3075) (end 125.9975 93.31) (width 0.3) (layer "F.Cu") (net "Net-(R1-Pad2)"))
 (segment (start 125.9975 93.31) (end 124.19 93.31) (width 0.3) (layer "F.Cu") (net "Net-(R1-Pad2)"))
 (segment (start 124.19 93.31) (end 124.18 93.3) (width 0.3) (layer "F.Cu") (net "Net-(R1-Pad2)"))
 (segment (start 126 90.98) (end 126 93.3075) (width 0.3) (layer "F.Cu") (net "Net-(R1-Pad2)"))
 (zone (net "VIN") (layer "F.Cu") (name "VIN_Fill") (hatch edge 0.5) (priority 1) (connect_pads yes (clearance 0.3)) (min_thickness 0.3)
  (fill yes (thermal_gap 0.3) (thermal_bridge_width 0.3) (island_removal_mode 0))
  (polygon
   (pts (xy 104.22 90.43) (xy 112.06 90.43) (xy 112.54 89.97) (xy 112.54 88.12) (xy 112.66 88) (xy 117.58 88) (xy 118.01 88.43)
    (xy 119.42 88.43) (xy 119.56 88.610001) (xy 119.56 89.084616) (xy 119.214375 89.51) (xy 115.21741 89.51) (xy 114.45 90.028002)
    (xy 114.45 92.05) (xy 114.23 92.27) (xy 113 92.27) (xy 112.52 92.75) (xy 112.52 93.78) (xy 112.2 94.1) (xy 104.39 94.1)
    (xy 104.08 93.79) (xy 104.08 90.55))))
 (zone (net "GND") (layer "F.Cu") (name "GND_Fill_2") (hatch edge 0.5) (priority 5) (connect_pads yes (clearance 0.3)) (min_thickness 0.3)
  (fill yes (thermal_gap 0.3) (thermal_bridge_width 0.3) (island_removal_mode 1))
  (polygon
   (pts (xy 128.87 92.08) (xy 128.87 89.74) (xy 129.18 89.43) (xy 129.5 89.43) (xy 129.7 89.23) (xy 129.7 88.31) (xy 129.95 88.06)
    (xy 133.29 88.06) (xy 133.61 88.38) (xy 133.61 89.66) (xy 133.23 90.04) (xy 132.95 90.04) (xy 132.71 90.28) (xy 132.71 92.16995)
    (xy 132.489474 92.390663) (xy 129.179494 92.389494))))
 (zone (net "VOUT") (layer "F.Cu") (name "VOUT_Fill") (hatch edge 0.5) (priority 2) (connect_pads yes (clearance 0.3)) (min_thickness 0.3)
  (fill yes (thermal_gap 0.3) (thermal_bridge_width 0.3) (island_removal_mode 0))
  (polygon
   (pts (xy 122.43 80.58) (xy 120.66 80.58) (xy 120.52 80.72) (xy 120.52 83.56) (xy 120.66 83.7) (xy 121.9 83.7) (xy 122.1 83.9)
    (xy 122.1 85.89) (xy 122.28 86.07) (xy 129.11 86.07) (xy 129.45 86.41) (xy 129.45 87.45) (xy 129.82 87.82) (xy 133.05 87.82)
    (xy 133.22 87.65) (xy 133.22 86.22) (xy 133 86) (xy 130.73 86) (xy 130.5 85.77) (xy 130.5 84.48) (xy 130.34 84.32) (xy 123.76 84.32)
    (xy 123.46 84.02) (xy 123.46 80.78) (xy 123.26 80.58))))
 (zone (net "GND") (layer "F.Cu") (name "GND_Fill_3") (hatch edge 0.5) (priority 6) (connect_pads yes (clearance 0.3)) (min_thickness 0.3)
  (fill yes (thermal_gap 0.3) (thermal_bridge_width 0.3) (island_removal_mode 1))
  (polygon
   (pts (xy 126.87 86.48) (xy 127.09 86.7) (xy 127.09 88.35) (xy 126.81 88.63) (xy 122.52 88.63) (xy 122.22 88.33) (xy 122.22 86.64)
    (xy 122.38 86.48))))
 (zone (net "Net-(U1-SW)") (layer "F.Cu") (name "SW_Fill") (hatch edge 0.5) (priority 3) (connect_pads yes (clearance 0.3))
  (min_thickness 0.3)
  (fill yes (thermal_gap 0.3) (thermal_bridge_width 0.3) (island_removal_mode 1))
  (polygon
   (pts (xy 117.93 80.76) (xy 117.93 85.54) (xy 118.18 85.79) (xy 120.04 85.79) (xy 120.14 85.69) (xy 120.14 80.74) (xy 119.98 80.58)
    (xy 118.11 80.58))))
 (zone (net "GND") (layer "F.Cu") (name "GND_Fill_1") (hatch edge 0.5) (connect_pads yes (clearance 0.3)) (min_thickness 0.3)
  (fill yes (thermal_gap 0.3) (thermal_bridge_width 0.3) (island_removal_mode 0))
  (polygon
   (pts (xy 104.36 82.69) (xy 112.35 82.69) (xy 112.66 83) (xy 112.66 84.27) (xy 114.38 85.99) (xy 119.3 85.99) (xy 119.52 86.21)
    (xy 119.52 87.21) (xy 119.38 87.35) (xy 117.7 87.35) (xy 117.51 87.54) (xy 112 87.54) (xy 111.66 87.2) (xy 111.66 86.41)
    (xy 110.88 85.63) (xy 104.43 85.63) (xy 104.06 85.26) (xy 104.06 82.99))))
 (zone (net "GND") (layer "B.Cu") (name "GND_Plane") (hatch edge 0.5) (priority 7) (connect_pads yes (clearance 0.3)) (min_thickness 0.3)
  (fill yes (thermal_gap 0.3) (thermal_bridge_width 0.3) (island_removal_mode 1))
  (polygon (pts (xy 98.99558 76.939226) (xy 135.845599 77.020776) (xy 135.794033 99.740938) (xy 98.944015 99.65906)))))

